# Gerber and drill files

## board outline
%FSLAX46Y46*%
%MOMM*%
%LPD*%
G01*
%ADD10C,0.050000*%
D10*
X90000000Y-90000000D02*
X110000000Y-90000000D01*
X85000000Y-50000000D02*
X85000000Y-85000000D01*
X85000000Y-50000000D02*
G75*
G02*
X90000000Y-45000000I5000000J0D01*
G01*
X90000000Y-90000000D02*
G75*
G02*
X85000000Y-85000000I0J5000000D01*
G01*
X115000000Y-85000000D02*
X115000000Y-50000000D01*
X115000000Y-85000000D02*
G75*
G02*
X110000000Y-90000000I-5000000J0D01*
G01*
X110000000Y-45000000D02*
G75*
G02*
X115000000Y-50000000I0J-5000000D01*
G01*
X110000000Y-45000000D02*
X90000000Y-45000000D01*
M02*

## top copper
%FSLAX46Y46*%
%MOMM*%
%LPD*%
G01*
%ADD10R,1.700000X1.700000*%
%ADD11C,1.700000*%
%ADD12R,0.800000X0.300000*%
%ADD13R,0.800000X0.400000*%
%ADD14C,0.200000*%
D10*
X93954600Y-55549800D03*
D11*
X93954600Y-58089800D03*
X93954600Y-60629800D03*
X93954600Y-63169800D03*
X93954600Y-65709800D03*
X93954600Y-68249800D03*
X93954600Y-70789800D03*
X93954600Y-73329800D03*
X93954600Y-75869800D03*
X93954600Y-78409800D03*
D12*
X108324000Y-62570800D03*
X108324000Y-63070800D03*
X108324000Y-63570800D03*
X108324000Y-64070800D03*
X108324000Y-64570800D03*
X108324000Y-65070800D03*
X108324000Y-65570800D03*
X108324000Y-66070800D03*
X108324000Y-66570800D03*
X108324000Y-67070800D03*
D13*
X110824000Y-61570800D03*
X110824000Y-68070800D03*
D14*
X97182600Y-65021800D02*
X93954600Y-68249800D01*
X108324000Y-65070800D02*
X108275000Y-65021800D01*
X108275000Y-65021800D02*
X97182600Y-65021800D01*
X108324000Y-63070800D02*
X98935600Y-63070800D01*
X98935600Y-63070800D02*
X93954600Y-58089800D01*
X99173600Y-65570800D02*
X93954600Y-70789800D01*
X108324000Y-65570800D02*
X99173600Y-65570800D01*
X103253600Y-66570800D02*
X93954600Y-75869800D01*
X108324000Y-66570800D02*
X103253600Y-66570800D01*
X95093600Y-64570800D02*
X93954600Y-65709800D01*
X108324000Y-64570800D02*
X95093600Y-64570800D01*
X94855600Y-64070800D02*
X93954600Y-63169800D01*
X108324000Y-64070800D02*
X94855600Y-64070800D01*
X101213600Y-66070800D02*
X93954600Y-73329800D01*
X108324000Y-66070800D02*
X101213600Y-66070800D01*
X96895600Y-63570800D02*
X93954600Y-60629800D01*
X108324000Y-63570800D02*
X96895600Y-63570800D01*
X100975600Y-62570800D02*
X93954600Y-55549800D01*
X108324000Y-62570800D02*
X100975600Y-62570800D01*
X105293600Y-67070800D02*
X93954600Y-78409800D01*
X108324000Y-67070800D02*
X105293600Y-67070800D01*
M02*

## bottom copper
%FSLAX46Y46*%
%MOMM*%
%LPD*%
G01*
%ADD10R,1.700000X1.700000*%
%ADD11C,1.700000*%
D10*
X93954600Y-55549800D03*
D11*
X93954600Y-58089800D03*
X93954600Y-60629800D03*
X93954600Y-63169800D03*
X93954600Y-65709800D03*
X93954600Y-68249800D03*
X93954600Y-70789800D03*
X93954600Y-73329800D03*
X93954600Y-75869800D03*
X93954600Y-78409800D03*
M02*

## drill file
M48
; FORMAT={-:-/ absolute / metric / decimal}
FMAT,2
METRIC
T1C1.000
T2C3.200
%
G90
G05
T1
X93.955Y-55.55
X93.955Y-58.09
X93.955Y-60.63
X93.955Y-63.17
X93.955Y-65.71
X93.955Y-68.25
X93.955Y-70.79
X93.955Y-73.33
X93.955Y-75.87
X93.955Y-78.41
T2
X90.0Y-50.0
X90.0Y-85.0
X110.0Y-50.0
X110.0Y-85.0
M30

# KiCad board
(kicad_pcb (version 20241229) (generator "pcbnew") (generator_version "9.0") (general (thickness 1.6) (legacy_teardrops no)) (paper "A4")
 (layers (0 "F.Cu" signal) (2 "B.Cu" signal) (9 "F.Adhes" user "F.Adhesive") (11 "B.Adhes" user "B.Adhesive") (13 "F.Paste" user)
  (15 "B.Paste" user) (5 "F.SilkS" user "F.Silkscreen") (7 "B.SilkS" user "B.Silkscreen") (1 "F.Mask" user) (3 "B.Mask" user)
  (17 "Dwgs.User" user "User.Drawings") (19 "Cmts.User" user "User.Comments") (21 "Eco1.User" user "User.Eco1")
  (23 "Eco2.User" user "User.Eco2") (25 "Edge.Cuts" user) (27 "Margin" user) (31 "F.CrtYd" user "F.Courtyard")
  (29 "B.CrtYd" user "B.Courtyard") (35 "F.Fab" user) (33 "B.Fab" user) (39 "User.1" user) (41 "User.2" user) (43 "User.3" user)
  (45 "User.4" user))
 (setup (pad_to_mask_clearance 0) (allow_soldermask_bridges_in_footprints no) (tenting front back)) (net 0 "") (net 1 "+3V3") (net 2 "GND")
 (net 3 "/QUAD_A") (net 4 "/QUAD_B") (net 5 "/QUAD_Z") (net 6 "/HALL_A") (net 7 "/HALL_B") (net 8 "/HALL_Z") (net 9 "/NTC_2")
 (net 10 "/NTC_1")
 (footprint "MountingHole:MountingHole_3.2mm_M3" (layer "F.Cu") (at 110 85)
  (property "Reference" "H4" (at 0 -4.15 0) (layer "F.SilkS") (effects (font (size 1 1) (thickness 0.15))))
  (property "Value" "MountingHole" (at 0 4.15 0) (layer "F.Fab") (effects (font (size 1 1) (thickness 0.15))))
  (pad "" np_thru_hole circle (at 0 0) (size 3.2 3.2) (drill 3.2) (layers "*.Cu" "*.Mask")))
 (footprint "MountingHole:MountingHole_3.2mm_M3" (layer "F.Cu") (at 90 85)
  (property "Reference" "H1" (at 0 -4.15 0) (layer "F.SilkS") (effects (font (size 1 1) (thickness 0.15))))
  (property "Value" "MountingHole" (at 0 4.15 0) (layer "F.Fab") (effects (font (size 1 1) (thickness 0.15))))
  (pad "" np_thru_hole circle (at 0 0) (size 3.2 3.2) (drill 3.2) (layers "*.Cu" "*.Mask")))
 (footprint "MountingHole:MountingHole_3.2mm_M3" (layer "F.Cu") (at 90 50)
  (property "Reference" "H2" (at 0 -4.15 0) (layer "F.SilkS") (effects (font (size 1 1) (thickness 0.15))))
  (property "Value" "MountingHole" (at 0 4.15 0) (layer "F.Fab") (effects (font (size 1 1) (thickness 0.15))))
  (pad "" np_thru_hole circle (at 0 0) (size 3.2 3.2) (drill 3.2) (layers "*.Cu" "*.Mask")))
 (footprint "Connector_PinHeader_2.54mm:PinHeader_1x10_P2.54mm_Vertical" (layer "F.Cu") (at 93.9546 55.5498)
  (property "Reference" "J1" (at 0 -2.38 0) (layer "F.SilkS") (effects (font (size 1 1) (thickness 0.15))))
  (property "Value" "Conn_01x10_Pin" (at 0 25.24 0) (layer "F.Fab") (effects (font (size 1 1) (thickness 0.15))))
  (pad "1" thru_hole rect (at 0 0) (size 1.7 1.7) (drill 1) (layers "*.Cu" "*.Mask") (remove_unused_layers no) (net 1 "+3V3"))
  (pad "2" thru_hole circle (at 0 2.54) (size 1.7 1.7) (drill 1) (layers "*.Cu" "*.Mask") (remove_unused_layers no) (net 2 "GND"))
  (pad "3" thru_hole circle (at 0 5.08) (size 1.7 1.7) (drill 1) (layers "*.Cu" "*.Mask") (remove_unused_layers no) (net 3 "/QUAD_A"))
  (pad "4" thru_hole circle (at 0 7.62) (size 1.7 1.7) (drill 1) (layers "*.Cu" "*.Mask") (remove_unused_layers no) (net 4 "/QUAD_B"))
  (pad "5" thru_hole circle (at 0 10.16) (size 1.7 1.7) (drill 1) (layers "*.Cu" "*.Mask") (remove_unused_layers no) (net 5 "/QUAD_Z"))
  (pad "6" thru_hole circle (at 0 12.7) (size 1.7 1.7) (drill 1) (layers "*.Cu" "*.Mask") (remove_unused_layers no) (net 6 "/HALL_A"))
  (pad "7" thru_hole circle (at 0 15.24) (size 1.7 1.7) (drill 1) (layers "*.Cu" "*.Mask") (remove_unused_layers no) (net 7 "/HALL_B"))
  (pad "8" thru_hole circle (at 0 17.78) (size 1.7 1.7) (drill 1) (layers "*.Cu" "*.Mask") (remove_unused_layers no) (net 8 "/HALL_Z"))
  (pad "9" thru_hole circle (at 0 20.32) (size 1.7 1.7) (drill 1) (layers "*.Cu" "*.Mask") (remove_unused_layers no) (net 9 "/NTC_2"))
  (pad "10" thru_hole circle (at 0 22.86) (size 1.7 1.7) (drill 1) (layers "*.Cu" "*.Mask") (remove_unused_layers no) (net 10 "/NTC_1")))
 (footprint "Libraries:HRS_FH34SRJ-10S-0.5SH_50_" (layer "F.Cu") (at 109.474 64.8208 90)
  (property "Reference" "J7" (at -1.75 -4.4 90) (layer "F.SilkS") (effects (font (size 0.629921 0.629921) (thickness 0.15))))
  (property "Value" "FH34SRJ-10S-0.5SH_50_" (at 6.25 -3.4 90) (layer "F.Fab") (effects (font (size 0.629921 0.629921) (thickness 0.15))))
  (pad "1" smd rect (at 2.25 -1.15 90) (size 0.3 0.8) (layers "F.Cu") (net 1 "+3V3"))
  (pad "2" smd rect (at 1.75 -1.15 90) (size 0.3 0.8) (layers "F.Cu") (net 2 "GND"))
  (pad "3" smd rect (at 1.25 -1.15 90) (size 0.3 0.8) (layers "F.Cu") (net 3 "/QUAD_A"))
  (pad "4" smd rect (at 0.75 -1.15 90) (size 0.3 0.8) (layers "F.Cu") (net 4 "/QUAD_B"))
  (pad "5" smd rect (at 0.25 -1.15 90) (size 0.3 0.8) (layers "F.Cu") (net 5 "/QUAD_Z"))
  (pad "6" smd rect (at -0.25 -1.15 90) (size 0.3 0.8) (layers "F.Cu") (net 6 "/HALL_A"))
  (pad "7" smd rect (at -0.75 -1.15 90) (size 0.3 0.8) (layers "F.Cu") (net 7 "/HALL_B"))
  (pad "8" smd rect (at -1.25 -1.15 90) (size 0.3 0.8) (layers "F.Cu") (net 8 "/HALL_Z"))
  (pad "9" smd rect (at -1.75 -1.15 90) (size 0.3 0.8) (layers "F.Cu") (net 9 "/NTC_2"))
  (pad "10" smd rect (at -2.25 -1.15 90) (size 0.3 0.8) (layers "F.Cu") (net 10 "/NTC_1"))
  (pad "S1" smd rect (at 3.25 1.35 90) (size 0.4 0.8) (layers "F.Cu" "F.Mask" "F.Paste") (solder_mask_margin 0.102))
  (pad "S2" smd rect (at -3.25 1.35 90) (size 0.4 0.8) (layers "F.Cu" "F.Mask" "F.Paste") (solder_mask_margin 0.102)))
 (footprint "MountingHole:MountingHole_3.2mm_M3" (layer "F.Cu") (at 110 50)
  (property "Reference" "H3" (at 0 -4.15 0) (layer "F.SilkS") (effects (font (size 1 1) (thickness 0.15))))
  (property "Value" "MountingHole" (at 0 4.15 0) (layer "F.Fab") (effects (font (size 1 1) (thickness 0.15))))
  (pad "" np_thru_hole circle (at 0 0) (size 3.2 3.2) (drill 3.2) (layers "*.Cu" "*.Mask")))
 (gr_line (start 90 90) (end 110 90) (stroke (width 0.05) (type default)) (layer "Edge.Cuts"))
 (gr_line (start 85 50) (end 85 85) (stroke (width 0.05) (type default)) (layer "Edge.Cuts"))
 (gr_arc (start 85 50) (mid 86.464466 46.464466) (end 90 45) (stroke (width 0.05) (type solid)) (layer "Edge.Cuts"))
 (gr_arc (start 90 90) (mid 86.464466 88.535534) (end 85 85) (stroke (width 0.05) (type solid)) (layer "Edge.Cuts"))
 (gr_line (start 115 85) (end 115 50) (stroke (width 0.05) (type default)) (layer "Edge.Cuts"))
 (gr_arc (start 115 85) (mid 113.535534 88.535534) (end 110 90) (stroke (width 0.05) (type solid)) (layer "Edge.Cuts"))
 (gr_arc (start 110 45) (mid 113.535534 46.464466) (end 115 50) (stroke (width 0.05) (type solid)) (layer "Edge.Cuts"))
 (gr_line (start 110 45) (end 90 45) (stroke (width 0.05) (type default)) (layer "Edge.Cuts"))
 (segment (start 97.1826 65.0218) (end 93.9546 68.2498) (width 0.2) (layer "F.Cu") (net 6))
 (segment (start 108.324 65.0708) (end 108.275 65.0218) (width 0.2) (layer "F.Cu") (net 6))
 (segment (start 108.275 65.0218) (end 97.1826 65.0218) (width 0.2) (layer "F.Cu") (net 6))
 (segment (start 108.324 63.0708) (end 98.9356 63.0708) (width 0.2) (layer "F.Cu") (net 2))
 (segment (start 98.9356 63.0708) (end 93.9546 58.0898) (width 0.2) (layer "F.Cu") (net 2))
 (segment (start 99.1736 65.5708) (end 93.9546 70.7898) (width 0.2) (layer "F.Cu") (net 7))
 (segment (start 108.324 65.5708) (end 99.1736 65.5708) (width 0.2) (layer "F.Cu") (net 7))
 (segment (start 103.2536 66.5708) (end 93.9546 75.8698) (width 0.2) (layer "F.Cu") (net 9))
 (segment (start 108.324 66.5708) (end 103.2536 66.5708) (width 0.2) (layer "F.Cu") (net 9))
 (segment (start 95.0936 64.5708) (end 93.9546 65.7098) (width 0.2) (layer "F.Cu") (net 5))
 (segment (start 108.324 64.5708) (end 95.0936 64.5708) (width 0.2) (layer "F.Cu") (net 5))
 (segment (start 94.8556 64.0708) (end 93.9546 63.1698) (width 0.2) (layer "F.Cu") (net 4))
 (segment (start 108.324 64.0708) (end 94.8556 64.0708) (width 0.2) (layer "F.Cu") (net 4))
 (segment (start 101.2136 66.0708) (end 93.9546 73.3298) (width 0.2) (layer "F.Cu") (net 8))
 (segment (start 108.324 66.0708) (end 101.2136 66.0708) (width 0.2) (layer "F.Cu") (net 8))
 (segment (start 96.8956 63.5708) (end 93.9546 60.6298) (width 0.2) (layer "F.Cu") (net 3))
 (segment (start 108.324 63.5708) (end 96.8956 63.5708) (width 0.2) (layer "F.Cu") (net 3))
 (segment (start 100.9756 62.5708) (end 93.9546 55.5498) (width 0.2) (layer "F.Cu") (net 1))
 (segment (start 108.324 62.5708) (end 100.9756 62.5708) (width 0.2) (layer "F.Cu") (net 1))
 (segment (start 105.2936 67.0708) (end 93.9546 78.4098) (width 0.2) (layer "F.Cu") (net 10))
 (segment (start 108.324 67.0708) (end 105.2936 67.0708) (width 0.2) (layer "F.Cu") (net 10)))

